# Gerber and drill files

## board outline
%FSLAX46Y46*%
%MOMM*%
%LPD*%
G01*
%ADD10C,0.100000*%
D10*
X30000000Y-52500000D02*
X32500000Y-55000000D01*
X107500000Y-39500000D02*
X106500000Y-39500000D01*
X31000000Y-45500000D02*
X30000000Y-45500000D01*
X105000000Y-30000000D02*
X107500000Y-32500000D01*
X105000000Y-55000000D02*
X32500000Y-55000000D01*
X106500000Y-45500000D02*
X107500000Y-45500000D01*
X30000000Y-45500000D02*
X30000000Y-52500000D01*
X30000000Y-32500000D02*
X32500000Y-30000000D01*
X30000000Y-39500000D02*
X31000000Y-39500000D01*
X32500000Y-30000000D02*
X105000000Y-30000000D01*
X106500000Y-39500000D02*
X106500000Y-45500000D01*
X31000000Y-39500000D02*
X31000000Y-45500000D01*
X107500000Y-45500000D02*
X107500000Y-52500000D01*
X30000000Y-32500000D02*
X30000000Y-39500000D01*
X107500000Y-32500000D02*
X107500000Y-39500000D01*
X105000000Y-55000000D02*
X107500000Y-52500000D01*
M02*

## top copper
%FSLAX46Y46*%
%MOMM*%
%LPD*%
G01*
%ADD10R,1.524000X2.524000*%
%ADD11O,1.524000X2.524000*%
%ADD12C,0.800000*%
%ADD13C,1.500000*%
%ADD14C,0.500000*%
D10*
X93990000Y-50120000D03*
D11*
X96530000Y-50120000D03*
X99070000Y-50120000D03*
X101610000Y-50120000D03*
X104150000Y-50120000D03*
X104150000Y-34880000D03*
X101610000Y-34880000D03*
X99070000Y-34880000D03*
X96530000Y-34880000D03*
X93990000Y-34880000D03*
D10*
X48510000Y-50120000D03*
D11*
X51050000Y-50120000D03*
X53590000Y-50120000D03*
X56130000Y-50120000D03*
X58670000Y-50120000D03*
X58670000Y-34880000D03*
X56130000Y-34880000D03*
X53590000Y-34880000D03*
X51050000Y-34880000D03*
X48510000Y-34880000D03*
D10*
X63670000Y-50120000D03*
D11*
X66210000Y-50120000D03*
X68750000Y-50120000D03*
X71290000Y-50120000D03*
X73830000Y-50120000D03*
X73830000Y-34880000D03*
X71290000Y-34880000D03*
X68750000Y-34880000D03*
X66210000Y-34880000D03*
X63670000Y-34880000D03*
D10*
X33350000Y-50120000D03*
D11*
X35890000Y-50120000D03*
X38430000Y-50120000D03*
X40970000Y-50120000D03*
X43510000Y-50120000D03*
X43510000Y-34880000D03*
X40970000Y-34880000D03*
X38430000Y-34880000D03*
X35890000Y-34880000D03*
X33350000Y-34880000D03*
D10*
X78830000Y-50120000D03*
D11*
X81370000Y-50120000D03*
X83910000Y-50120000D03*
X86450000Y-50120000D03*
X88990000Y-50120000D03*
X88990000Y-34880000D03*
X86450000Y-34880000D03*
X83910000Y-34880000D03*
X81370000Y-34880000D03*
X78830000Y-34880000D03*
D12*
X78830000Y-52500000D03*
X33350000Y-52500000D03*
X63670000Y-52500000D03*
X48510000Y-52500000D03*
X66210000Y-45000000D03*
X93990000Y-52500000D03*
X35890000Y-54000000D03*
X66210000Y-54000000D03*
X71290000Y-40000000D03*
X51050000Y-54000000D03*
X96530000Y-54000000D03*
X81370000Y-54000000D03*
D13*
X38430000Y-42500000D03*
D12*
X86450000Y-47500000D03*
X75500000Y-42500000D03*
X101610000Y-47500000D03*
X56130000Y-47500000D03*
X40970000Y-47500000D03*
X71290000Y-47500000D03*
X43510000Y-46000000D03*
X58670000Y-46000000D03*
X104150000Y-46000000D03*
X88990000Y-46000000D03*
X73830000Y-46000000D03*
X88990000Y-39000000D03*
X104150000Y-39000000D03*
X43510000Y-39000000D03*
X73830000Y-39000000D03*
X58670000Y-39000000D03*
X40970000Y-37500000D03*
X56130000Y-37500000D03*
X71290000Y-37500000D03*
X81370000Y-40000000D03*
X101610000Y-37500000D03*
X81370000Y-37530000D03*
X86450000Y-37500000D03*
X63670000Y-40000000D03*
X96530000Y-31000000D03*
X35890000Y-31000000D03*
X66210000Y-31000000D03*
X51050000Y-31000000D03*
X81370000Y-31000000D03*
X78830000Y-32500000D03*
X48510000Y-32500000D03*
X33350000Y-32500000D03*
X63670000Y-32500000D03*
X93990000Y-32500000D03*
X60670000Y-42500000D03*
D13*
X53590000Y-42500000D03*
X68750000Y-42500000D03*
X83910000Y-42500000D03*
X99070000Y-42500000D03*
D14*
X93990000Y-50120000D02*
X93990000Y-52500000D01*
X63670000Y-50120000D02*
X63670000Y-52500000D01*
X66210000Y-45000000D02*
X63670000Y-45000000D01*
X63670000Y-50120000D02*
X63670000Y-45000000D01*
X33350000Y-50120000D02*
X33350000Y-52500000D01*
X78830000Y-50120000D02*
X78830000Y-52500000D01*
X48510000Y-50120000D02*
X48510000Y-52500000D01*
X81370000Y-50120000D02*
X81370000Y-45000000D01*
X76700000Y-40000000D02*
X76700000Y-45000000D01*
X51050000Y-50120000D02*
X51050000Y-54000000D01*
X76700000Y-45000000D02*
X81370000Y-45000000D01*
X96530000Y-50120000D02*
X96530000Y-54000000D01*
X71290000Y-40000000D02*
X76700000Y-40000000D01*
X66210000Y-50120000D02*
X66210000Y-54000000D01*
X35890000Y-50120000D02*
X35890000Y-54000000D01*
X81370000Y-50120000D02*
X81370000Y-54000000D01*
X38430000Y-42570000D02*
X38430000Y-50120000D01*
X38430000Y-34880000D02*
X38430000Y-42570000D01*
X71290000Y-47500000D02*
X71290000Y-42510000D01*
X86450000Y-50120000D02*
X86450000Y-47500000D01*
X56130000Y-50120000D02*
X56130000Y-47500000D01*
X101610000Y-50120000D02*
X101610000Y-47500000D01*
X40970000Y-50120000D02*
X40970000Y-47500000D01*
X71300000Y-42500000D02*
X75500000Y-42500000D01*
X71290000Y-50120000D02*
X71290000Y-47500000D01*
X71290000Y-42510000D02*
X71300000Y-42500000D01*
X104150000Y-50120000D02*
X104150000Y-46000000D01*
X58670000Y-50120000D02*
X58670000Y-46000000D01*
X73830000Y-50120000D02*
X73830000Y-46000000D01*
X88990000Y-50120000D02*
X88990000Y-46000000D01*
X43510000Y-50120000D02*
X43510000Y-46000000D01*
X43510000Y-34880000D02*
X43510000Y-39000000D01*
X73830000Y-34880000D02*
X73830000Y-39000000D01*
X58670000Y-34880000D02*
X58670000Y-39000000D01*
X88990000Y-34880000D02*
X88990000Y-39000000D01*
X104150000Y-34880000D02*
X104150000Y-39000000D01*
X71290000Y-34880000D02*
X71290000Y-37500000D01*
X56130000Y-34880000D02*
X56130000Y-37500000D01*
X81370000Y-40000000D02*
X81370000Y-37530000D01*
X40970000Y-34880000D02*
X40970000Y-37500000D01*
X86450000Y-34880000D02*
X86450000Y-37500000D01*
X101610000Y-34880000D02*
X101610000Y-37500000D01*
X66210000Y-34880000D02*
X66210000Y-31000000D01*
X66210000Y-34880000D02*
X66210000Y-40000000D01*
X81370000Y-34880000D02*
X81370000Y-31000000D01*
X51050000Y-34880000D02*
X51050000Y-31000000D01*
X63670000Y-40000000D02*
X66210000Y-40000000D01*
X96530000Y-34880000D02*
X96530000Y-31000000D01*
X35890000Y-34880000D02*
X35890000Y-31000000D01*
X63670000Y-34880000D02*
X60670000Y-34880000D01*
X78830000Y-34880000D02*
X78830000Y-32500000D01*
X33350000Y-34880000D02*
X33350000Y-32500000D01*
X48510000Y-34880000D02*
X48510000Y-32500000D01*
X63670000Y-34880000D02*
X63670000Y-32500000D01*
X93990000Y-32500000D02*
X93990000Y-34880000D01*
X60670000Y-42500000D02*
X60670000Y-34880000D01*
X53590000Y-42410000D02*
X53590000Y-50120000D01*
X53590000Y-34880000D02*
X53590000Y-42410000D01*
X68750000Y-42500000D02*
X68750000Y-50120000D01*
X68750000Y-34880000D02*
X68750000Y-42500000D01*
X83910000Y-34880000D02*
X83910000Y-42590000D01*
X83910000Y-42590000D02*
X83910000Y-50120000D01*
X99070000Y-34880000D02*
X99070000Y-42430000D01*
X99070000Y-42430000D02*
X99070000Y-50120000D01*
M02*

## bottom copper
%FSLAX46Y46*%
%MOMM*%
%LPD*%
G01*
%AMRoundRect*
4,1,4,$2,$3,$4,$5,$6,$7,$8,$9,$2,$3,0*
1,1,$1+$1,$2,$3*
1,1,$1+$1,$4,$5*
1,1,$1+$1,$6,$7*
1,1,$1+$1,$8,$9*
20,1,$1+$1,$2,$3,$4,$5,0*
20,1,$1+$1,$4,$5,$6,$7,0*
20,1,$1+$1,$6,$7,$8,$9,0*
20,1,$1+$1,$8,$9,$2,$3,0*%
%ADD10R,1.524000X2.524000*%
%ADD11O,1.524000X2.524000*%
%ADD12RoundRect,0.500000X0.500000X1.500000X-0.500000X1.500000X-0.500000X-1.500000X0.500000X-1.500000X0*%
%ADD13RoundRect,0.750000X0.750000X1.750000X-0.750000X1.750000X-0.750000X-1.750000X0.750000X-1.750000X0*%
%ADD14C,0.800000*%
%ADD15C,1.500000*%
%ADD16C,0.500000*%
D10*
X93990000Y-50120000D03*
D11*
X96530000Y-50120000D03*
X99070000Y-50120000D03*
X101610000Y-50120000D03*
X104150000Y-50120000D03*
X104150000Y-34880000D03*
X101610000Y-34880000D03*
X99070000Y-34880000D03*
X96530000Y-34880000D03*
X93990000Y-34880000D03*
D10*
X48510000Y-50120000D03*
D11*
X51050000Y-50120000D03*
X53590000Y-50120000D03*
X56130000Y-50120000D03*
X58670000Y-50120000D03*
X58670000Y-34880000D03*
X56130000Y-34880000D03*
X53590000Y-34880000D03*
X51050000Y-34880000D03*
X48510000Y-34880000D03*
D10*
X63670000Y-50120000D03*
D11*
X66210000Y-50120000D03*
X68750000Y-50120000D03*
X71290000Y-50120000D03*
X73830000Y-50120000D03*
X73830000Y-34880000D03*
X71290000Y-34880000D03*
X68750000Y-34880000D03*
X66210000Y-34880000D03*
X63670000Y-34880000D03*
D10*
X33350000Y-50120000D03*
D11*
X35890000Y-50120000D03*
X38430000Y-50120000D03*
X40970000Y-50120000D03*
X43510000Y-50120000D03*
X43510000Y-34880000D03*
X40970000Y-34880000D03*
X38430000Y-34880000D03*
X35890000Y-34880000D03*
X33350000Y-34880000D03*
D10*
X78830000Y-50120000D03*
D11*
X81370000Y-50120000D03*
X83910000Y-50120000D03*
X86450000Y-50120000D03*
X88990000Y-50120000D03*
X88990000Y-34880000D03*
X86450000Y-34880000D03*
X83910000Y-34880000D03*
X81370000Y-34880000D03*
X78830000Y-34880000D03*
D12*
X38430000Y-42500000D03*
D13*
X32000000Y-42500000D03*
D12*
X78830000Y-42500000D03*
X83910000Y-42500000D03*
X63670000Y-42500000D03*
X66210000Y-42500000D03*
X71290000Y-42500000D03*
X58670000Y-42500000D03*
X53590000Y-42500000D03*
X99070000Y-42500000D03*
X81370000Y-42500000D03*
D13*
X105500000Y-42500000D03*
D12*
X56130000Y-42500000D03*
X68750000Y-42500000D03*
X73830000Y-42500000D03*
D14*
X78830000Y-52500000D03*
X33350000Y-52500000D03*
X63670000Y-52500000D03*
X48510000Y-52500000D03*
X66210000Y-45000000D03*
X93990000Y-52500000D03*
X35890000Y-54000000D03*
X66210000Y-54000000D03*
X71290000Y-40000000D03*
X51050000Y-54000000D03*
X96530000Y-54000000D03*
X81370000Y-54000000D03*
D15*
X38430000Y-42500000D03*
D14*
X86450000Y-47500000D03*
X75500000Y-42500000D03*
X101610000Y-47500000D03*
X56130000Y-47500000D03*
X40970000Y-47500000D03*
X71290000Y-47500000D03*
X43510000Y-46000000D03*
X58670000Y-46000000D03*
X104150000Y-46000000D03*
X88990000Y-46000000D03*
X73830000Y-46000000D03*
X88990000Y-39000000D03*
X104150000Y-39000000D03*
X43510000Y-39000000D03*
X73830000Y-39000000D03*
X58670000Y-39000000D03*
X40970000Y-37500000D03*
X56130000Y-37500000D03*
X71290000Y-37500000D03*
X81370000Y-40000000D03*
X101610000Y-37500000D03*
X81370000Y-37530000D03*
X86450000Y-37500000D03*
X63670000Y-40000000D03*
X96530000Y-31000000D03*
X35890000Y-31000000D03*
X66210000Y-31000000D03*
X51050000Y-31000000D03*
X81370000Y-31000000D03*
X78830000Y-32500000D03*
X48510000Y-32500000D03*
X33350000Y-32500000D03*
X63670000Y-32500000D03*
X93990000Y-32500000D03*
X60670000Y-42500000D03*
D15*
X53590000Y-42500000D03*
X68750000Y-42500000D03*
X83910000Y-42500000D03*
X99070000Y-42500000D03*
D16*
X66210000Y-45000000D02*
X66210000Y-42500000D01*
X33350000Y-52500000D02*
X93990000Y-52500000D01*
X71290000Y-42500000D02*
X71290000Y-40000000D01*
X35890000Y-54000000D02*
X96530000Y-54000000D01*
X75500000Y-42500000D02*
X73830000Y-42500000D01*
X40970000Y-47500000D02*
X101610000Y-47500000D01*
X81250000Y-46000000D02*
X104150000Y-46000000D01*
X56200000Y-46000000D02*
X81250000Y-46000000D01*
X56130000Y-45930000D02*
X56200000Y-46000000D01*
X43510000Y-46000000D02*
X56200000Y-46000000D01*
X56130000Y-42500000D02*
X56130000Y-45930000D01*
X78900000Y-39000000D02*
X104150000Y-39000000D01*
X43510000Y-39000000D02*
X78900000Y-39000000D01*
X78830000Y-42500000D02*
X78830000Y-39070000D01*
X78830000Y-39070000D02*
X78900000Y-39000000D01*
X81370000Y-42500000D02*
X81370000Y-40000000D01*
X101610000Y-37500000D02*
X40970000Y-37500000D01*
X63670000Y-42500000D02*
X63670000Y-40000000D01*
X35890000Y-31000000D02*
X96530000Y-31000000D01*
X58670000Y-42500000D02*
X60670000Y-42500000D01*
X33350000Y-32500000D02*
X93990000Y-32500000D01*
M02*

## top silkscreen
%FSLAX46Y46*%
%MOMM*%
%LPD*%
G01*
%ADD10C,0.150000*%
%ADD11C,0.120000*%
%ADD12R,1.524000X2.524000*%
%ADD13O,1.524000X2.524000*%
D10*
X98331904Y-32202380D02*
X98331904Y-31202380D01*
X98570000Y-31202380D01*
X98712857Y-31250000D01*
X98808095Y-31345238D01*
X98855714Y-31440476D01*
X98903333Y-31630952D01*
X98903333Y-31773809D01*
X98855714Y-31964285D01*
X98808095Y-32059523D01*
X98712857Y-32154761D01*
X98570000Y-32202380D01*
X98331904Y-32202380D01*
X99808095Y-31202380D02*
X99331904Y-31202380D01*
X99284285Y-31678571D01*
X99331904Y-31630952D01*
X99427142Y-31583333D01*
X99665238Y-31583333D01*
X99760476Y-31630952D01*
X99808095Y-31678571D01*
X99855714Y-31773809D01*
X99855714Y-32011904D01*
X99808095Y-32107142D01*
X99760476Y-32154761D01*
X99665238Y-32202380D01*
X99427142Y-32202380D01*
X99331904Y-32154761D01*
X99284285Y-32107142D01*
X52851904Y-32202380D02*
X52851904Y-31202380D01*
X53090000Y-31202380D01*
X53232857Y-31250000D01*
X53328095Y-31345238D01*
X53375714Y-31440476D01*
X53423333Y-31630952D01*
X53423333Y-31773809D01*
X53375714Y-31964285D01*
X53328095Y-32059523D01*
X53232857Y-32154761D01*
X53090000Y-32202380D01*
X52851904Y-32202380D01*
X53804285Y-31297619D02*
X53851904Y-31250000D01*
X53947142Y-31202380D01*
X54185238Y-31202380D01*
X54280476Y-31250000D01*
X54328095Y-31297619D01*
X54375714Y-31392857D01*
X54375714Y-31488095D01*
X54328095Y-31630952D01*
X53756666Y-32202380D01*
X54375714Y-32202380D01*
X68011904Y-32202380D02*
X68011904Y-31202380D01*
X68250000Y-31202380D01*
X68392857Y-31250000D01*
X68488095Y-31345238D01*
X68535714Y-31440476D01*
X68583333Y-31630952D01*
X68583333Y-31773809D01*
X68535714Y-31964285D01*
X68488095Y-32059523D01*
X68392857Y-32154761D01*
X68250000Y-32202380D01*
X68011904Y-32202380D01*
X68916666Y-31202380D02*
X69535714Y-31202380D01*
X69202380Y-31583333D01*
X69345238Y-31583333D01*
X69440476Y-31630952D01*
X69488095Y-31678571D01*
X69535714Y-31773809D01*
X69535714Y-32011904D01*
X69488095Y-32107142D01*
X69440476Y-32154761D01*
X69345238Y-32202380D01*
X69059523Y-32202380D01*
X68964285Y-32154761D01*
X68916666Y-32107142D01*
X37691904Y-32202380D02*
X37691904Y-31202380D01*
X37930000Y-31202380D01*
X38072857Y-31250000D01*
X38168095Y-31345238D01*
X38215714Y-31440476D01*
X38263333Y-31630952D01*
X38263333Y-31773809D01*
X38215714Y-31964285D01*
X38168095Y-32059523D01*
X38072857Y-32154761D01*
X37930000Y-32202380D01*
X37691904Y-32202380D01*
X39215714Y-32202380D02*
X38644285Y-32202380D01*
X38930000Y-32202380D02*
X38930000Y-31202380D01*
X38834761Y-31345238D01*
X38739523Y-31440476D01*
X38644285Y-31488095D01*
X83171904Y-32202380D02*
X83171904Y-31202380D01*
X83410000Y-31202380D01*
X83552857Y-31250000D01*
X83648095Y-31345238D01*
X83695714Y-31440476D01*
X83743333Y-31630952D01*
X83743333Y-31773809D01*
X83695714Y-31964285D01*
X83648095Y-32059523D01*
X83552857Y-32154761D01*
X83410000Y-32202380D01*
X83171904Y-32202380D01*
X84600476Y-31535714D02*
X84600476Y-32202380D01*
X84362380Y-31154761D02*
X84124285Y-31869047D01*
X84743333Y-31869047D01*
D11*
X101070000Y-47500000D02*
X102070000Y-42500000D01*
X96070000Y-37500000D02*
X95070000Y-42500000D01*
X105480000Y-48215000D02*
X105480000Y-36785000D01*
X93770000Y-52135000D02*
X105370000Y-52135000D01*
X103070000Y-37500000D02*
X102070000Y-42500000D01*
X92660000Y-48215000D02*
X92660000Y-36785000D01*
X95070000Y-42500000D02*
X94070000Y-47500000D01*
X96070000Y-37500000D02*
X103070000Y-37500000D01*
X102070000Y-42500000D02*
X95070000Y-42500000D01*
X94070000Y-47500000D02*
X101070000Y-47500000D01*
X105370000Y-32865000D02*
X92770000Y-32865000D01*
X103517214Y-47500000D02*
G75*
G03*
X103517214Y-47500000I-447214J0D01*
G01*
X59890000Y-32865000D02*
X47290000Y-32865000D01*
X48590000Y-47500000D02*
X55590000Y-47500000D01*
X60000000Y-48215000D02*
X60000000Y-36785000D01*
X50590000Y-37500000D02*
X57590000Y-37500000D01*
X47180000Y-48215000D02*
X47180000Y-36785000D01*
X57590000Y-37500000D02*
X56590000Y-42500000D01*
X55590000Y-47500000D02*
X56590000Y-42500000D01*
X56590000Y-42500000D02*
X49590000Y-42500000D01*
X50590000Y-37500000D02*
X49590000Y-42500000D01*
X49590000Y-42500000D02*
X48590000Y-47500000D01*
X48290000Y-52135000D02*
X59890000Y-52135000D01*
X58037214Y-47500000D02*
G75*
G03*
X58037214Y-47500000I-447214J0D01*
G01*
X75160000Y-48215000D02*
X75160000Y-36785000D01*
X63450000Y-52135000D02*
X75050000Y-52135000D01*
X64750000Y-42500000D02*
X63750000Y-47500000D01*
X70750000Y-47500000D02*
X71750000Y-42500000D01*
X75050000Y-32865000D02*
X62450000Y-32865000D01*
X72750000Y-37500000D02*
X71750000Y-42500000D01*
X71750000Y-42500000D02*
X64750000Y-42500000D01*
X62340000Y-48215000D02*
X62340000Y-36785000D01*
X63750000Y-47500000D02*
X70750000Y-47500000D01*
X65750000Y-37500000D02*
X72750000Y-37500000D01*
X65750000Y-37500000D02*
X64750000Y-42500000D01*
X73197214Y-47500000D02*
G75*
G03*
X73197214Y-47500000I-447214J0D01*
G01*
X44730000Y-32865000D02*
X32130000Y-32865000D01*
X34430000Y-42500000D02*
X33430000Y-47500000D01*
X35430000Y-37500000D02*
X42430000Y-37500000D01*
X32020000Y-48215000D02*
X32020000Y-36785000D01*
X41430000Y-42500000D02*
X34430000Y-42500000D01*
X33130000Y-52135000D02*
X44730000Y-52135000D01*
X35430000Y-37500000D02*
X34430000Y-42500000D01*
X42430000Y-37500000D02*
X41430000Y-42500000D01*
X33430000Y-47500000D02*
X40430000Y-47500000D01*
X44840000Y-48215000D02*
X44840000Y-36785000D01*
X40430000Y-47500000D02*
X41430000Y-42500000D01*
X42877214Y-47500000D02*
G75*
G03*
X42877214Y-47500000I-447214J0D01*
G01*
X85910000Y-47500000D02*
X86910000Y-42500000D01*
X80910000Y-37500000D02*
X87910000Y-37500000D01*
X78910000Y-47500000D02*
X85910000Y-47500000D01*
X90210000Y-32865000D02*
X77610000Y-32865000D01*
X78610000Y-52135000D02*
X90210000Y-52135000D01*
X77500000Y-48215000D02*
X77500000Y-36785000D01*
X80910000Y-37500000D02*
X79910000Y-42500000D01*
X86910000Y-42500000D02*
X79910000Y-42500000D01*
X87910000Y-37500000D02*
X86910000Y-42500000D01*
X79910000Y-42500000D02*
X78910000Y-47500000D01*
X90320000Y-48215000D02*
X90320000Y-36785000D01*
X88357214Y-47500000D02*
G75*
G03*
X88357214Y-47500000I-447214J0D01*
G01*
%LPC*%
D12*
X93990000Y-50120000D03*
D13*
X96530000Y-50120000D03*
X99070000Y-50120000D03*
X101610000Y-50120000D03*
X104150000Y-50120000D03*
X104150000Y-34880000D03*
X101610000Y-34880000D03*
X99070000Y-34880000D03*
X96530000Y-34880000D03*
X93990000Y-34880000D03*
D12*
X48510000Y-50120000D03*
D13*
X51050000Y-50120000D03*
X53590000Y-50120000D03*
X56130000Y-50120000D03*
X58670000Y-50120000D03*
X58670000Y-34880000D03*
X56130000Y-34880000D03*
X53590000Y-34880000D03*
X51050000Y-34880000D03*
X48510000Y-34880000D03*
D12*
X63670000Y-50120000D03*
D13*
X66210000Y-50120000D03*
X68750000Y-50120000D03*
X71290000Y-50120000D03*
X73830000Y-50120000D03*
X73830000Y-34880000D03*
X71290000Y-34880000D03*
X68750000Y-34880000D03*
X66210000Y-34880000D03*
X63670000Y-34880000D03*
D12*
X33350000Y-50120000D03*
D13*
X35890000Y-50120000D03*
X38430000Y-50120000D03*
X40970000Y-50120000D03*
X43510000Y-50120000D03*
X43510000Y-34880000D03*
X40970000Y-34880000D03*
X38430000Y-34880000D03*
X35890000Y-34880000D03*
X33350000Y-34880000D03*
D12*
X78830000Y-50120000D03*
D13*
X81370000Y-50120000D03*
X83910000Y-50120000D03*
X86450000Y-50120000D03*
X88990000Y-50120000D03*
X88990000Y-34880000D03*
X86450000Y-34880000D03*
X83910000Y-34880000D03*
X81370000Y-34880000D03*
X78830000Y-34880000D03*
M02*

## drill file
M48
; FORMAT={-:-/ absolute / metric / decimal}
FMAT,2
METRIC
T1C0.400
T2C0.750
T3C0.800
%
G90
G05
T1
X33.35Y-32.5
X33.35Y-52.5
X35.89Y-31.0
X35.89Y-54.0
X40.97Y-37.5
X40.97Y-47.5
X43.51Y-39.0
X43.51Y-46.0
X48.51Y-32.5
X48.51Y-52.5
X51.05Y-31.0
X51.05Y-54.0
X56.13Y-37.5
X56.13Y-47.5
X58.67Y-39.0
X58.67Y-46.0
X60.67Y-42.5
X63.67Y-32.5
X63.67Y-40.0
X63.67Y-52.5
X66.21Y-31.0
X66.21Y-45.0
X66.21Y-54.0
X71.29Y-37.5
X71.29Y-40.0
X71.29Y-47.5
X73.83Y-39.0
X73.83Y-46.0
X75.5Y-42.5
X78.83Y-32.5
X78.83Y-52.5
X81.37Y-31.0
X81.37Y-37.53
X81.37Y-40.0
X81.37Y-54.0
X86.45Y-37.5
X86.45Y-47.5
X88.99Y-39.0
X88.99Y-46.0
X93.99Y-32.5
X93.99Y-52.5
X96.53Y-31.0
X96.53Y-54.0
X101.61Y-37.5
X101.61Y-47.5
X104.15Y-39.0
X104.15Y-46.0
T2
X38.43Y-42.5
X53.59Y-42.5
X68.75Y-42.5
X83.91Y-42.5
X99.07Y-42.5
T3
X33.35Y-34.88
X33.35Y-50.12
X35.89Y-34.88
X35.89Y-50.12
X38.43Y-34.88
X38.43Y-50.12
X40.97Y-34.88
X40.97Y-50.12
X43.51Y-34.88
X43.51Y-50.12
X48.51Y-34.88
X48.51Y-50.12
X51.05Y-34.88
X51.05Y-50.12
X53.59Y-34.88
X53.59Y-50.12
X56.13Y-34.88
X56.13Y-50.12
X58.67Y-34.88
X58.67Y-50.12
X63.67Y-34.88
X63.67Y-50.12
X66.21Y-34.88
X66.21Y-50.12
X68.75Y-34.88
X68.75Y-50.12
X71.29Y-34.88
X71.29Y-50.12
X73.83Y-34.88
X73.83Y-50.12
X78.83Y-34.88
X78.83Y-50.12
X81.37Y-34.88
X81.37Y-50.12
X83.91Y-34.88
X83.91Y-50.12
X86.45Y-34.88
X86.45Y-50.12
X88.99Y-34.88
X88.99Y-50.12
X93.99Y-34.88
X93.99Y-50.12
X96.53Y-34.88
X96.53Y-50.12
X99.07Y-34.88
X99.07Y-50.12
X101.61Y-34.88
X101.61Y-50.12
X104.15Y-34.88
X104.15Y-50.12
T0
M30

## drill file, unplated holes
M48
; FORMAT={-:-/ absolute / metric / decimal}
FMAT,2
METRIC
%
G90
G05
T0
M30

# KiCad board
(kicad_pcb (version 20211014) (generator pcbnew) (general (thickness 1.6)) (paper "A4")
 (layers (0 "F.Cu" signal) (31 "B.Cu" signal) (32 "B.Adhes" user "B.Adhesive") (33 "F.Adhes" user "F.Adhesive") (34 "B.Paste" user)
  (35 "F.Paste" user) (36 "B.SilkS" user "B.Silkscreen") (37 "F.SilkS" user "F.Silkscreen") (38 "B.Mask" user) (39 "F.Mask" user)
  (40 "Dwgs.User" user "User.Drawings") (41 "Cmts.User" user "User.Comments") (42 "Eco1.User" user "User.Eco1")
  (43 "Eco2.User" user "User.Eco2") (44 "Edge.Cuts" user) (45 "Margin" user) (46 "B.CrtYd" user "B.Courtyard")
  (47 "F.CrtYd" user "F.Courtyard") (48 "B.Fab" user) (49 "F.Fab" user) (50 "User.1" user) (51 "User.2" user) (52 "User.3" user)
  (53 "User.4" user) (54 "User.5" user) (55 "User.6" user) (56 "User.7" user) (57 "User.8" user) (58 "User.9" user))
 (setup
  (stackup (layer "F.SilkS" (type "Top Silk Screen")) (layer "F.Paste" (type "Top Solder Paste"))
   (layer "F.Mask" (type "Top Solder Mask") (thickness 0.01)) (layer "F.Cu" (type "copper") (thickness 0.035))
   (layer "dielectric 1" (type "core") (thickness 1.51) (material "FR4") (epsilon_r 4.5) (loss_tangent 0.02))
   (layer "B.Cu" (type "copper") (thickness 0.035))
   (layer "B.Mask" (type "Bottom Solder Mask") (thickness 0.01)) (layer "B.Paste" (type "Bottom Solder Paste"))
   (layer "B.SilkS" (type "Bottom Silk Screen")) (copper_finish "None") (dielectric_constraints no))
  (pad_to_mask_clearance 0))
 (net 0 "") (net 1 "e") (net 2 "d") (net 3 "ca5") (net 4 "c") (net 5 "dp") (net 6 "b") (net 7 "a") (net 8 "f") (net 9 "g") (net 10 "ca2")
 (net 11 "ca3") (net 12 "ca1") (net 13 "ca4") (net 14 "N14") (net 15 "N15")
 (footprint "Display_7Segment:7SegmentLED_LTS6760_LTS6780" (layer "F.Cu") (at 93.99 50.12 90)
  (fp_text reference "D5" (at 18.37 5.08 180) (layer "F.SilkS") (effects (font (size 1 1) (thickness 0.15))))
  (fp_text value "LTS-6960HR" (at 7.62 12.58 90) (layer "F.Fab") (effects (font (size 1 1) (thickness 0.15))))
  (fp_line (start 2.62 7.08) (end 7.62 8.08) (layer "F.SilkS") (width 0.12))
  (fp_line (start 12.62 2.08) (end 7.62 1.08) (layer "F.SilkS") (width 0.12))
  (fp_line (start 1.905 11.49) (end 13.335 11.49) (layer "F.SilkS") (width 0.12))
  (fp_line (start -2.015 -0.22) (end -2.015 11.38) (layer "F.SilkS") (width 0.12))
  (fp_line (start 12.62 9.08) (end 7.62 8.08) (layer "F.SilkS") (width 0.12))
  (fp_line (start 1.905 -1.33) (end 13.335 -1.33) (layer "F.SilkS") (width 0.12))
  (fp_line (start 7.62 1.08) (end 2.62 0.08) (layer "F.SilkS") (width 0.12))
  (fp_line (start 12.62 2.08) (end 12.62 9.08) (layer "F.SilkS") (width 0.12))
  (fp_line (start 7.62 8.08) (end 7.62 1.08) (layer "F.SilkS") (width 0.12))
  (fp_line (start 2.62 0.08) (end 2.62 7.08) (layer "F.SilkS") (width 0.12))
  (fp_line (start 17.255 11.38) (end 17.255 -1.22) (layer "F.SilkS") (width 0.12))
  (fp_circle (center 2.62 9.08) (end 3.067214 9.08) (layer "F.SilkS") (width 0.12) (fill none))
  (pad "1" thru_hole rect (at 0 0) (size 1.524 2.524) (drill 0.8) (layers *.Cu *.Mask) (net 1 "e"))
  (pad "2" thru_hole oval (at 0 2.54) (size 1.524 2.524) (drill 0.8) (layers *.Cu *.Mask) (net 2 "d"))
  (pad "3" thru_hole oval (at 0 5.08) (size 1.524 2.524) (drill 0.8) (layers *.Cu *.Mask) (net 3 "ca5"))
  (pad "4" thru_hole oval (at 0 7.62) (size 1.524 2.524) (drill 0.8) (layers *.Cu *.Mask) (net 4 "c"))
  (pad "5" thru_hole oval (at 0 10.16) (size 1.524 2.524) (drill 0.8) (layers *.Cu *.Mask) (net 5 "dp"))
  (pad "6" thru_hole oval (at 15.24 10.16) (size 1.524 2.524) (drill 0.8) (layers *.Cu *.Mask) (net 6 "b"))
  (pad "7" thru_hole oval (at 15.24 7.62) (size 1.524 2.524) (drill 0.8) (layers *.Cu *.Mask) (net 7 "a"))
  (pad "8" thru_hole oval (at 15.24 5.08) (size 1.524 2.524) (drill 0.8) (layers *.Cu *.Mask) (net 3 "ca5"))
  (pad "9" thru_hole oval (at 15.24 2.54) (size 1.524 2.524) (drill 0.8) (layers *.Cu *.Mask) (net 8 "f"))
  (pad "10" thru_hole oval (at 15.24 0) (size 1.524 2.524) (drill 0.8) (layers *.Cu *.Mask) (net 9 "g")))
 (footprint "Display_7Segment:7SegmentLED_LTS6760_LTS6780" (layer "F.Cu") (at 48.51 50.12 90)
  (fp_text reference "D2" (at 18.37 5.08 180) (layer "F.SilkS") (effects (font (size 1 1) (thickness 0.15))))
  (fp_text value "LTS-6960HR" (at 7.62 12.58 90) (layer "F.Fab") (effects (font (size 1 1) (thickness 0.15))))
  (fp_line (start 17.255 11.38) (end 17.255 -1.22) (layer "F.SilkS") (width 0.12))
  (fp_line (start 2.62 0.08) (end 2.62 7.08) (layer "F.SilkS") (width 0.12))
  (fp_line (start 1.905 11.49) (end 13.335 11.49) (layer "F.SilkS") (width 0.12))
  (fp_line (start 12.62 2.08) (end 12.62 9.08) (layer "F.SilkS") (width 0.12))
  (fp_line (start 1.905 -1.33) (end 13.335 -1.33) (layer "F.SilkS") (width 0.12))
  (fp_line (start 12.62 9.08) (end 7.62 8.08) (layer "F.SilkS") (width 0.12))
  (fp_line (start 2.62 7.08) (end 7.62 8.08) (layer "F.SilkS") (width 0.12))
  (fp_line (start 7.62 8.08) (end 7.62 1.08) (layer "F.SilkS") (width 0.12))
  (fp_line (start 12.62 2.08) (end 7.62 1.08) (layer "F.SilkS") (width 0.12))
  (fp_line (start 7.62 1.08) (end 2.62 0.08) (layer "F.SilkS") (width 0.12))
  (fp_line (start -2.015 -0.22) (end -2.015 11.38) (layer "F.SilkS") (width 0.12))
  (fp_circle (center 2.62 9.08) (end 3.067214 9.08) (layer "F.SilkS") (width 0.12) (fill none))
  (pad "1" thru_hole rect (at 0 0) (size 1.524 2.524) (drill 0.8) (layers *.Cu *.Mask) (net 1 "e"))
  (pad "2" thru_hole oval (at 0 2.54) (size 1.524 2.524) (drill 0.8) (layers *.Cu *.Mask) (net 2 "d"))
  (pad "3" thru_hole oval (at 0 5.08) (size 1.524 2.524) (drill 0.8) (layers *.Cu *.Mask) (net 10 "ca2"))
  (pad "4" thru_hole oval (at 0 7.62) (size 1.524 2.524) (drill 0.8) (layers *.Cu *.Mask) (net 4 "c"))
  (pad "5" thru_hole oval (at 0 10.16) (size 1.524 2.524) (drill 0.8) (layers *.Cu *.Mask) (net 5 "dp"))
  (pad "6" thru_hole oval (at 15.24 10.16) (size 1.524 2.524) (drill 0.8) (layers *.Cu *.Mask) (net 6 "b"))
  (pad "7" thru_hole oval (at 15.24 7.62) (size 1.524 2.524) (drill 0.8) (layers *.Cu *.Mask) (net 7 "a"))
  (pad "8" thru_hole oval (at 15.24 5.08) (size 1.524 2.524) (drill 0.8) (layers *.Cu *.Mask) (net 10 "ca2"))
  (pad "9" thru_hole oval (at 15.24 2.54) (size 1.524 2.524) (drill 0.8) (layers *.Cu *.Mask) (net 8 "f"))
  (pad "10" thru_hole oval (at 15.24 0) (size 1.524 2.524) (drill 0.8) (layers *.Cu *.Mask) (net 9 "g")))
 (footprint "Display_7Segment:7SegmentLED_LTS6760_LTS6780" (layer "F.Cu") (at 63.67 50.12 90)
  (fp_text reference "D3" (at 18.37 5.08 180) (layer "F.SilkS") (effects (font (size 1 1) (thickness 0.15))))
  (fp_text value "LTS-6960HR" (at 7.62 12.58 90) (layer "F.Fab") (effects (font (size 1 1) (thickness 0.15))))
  (fp_line (start 1.905 11.49) (end 13.335 11.49) (layer "F.SilkS") (width 0.12))
  (fp_line (start -2.015 -0.22) (end -2.015 11.38) (layer "F.SilkS") (width 0.12))
  (fp_line (start 7.62 1.08) (end 2.62 0.08) (layer "F.SilkS") (width 0.12))
  (fp_line (start 2.62 7.08) (end 7.62 8.08) (layer "F.SilkS") (width 0.12))
  (fp_line (start 17.255 11.38) (end 17.255 -1.22) (layer "F.SilkS") (width 0.12))
  (fp_line (start 12.62 9.08) (end 7.62 8.08) (layer "F.SilkS") (width 0.12))
  (fp_line (start 7.62 8.08) (end 7.62 1.08) (layer "F.SilkS") (width 0.12))
  (fp_line (start 1.905 -1.33) (end 13.335 -1.33) (layer "F.SilkS") (width 0.12))
  (fp_line (start 2.62 0.08) (end 2.62 7.08) (layer "F.SilkS") (width 0.12))
  (fp_line (start 12.62 2.08) (end 12.62 9.08) (layer "F.SilkS") (width 0.12))
  (fp_line (start 12.62 2.08) (end 7.62 1.08) (layer "F.SilkS") (width 0.12))
  (fp_circle (center 2.62 9.08) (end 3.067214 9.08) (layer "F.SilkS") (width 0.12) (fill none))
  (pad "1" thru_hole rect (at 0 0) (size 1.524 2.524) (drill 0.8) (layers *.Cu *.Mask) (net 1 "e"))
  (pad "2" thru_hole oval (at 0 2.54) (size 1.524 2.524) (drill 0.8) (layers *.Cu *.Mask) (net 2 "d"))
  (pad "3" thru_hole oval (at 0 5.08) (size 1.524 2.524) (drill 0.8) (layers *.Cu *.Mask) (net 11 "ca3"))
  (pad "4" thru_hole oval (at 0 7.62) (size 1.524 2.524) (drill 0.8) (layers *.Cu *.Mask) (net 4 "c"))
  (pad "5" thru_hole oval (at 0 10.16) (size 1.524 2.524) (drill 0.8) (layers *.Cu *.Mask) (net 5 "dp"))
  (pad "6" thru_hole oval (at 15.24 10.16) (size 1.524 2.524) (drill 0.8) (layers *.Cu *.Mask) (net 6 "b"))
  (pad "7" thru_hole oval (at 15.24 7.62) (size 1.524 2.524) (drill 0.8) (layers *.Cu *.Mask) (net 7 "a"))
  (pad "8" thru_hole oval (at 15.24 5.08) (size 1.524 2.524) (drill 0.8) (layers *.Cu *.Mask) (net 11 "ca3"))
  (pad "9" thru_hole oval (at 15.24 2.54) (size 1.524 2.524) (drill 0.8) (layers *.Cu *.Mask) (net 8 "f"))
  (pad "10" thru_hole oval (at 15.24 0) (size 1.524 2.524) (drill 0.8) (layers *.Cu *.Mask) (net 9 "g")))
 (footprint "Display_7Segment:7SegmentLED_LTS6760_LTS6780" (layer "F.Cu") (at 33.35 50.12 90)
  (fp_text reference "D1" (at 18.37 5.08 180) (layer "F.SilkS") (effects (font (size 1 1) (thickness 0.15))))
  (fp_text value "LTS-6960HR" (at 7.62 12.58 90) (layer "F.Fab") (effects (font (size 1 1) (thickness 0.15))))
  (fp_line (start 17.255 11.38) (end 17.255 -1.22) (layer "F.SilkS") (width 0.12))
  (fp_line (start 7.62 1.08) (end 2.62 0.08) (layer "F.SilkS") (width 0.12))
  (fp_line (start 12.62 2.08) (end 12.62 9.08) (layer "F.SilkS") (width 0.12))
  (fp_line (start 1.905 -1.33) (end 13.335 -1.33) (layer "F.SilkS") (width 0.12))
  (fp_line (start 7.62 8.08) (end 7.62 1.08) (layer "F.SilkS") (width 0.12))
  (fp_line (start -2.015 -0.22) (end -2.015 11.38) (layer "F.SilkS") (width 0.12))
  (fp_line (start 12.62 2.08) (end 7.62 1.08) (layer "F.SilkS") (width 0.12))
  (fp_line (start 12.62 9.08) (end 7.62 8.08) (layer "F.SilkS") (width 0.12))
  (fp_line (start 2.62 0.08) (end 2.62 7.08) (layer "F.SilkS") (width 0.12))
  (fp_line (start 1.905 11.49) (end 13.335 11.49) (layer "F.SilkS") (width 0.12))
  (fp_line (start 2.62 7.08) (end 7.62 8.08) (layer "F.SilkS") (width 0.12))
  (fp_circle (center 2.62 9.08) (end 3.067214 9.08) (layer "F.SilkS") (width 0.12) (fill none))
  (pad "1" thru_hole rect (at 0 0) (size 1.524 2.524) (drill 0.8) (layers *.Cu *.Mask) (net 1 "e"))
  (pad "2" thru_hole oval (at 0 2.54) (size 1.524 2.524) (drill 0.8) (layers *.Cu *.Mask) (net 2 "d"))
  (pad "3" thru_hole oval (at 0 5.08) (size 1.524 2.524) (drill 0.8) (layers *.Cu *.Mask) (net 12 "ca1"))
  (pad "4" thru_hole oval (at 0 7.62) (size 1.524 2.524) (drill 0.8) (layers *.Cu *.Mask) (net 4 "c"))
  (pad "5" thru_hole oval (at 0 10.16) (size 1.524 2.524) (drill 0.8) (layers *.Cu *.Mask) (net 5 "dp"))
  (pad "6" thru_hole oval (at 15.24 10.16) (size 1.524 2.524) (drill 0.8) (layers *.Cu *.Mask) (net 6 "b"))
  (pad "7" thru_hole oval (at 15.24 7.62) (size 1.524 2.524) (drill 0.8) (layers *.Cu *.Mask) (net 7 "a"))
  (pad "8" thru_hole oval (at 15.24 5.08) (size 1.524 2.524) (drill 0.8) (layers *.Cu *.Mask) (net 12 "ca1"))
  (pad "9" thru_hole oval (at 15.24 2.54) (size 1.524 2.524) (drill 0.8) (layers *.Cu *.Mask) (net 8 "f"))
  (pad "10" thru_hole oval (at 15.24 0) (size 1.524 2.524) (drill 0.8) (layers *.Cu *.Mask) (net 9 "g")))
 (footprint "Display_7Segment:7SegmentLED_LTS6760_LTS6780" (layer "F.Cu") (at 78.83 50.12 90)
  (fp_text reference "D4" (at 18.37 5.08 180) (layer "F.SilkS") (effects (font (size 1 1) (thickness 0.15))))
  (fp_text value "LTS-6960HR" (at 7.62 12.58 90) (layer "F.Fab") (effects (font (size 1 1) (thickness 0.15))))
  (fp_line (start 2.62 7.08) (end 7.62 8.08) (layer "F.SilkS") (width 0.12))
  (fp_line (start 12.62 2.08) (end 12.62 9.08) (layer "F.SilkS") (width 0.12))
  (fp_line (start 2.62 0.08) (end 2.62 7.08) (layer "F.SilkS") (width 0.12))
  (fp_line (start 17.255 11.38) (end 17.255 -1.22) (layer "F.SilkS") (width 0.12))
  (fp_line (start -2.015 -0.22) (end -2.015 11.38) (layer "F.SilkS") (width 0.12))
  (fp_line (start 1.905 -1.33) (end 13.335 -1.33) (layer "F.SilkS") (width 0.12))
  (fp_line (start 12.62 2.08) (end 7.62 1.08) (layer "F.SilkS") (width 0.12))
  (fp_line (start 7.62 8.08) (end 7.62 1.08) (layer "F.SilkS") (width 0.12))
  (fp_line (start 12.62 9.08) (end 7.62 8.08) (layer "F.SilkS") (width 0.12))
  (fp_line (start 7.62 1.08) (end 2.62 0.08) (layer "F.SilkS") (width 0.12))
  (fp_line (start 1.905 11.49) (end 13.335 11.49) (layer "F.SilkS") (width 0.12))
  (fp_circle (center 2.62 9.08) (end 3.067214 9.08) (layer "F.SilkS") (width 0.12) (fill none))
  (pad "1" thru_hole rect (at 0 0) (size 1.524 2.524) (drill 0.8) (layers *.Cu *.Mask) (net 1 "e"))
  (pad "2" thru_hole oval (at 0 2.54) (size 1.524 2.524) (drill 0.8) (layers *.Cu *.Mask) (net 2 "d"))
  (pad "3" thru_hole oval (at 0 5.08) (size 1.524 2.524) (drill 0.8) (layers *.Cu *.Mask) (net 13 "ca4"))
  (pad "4" thru_hole oval (at 0 7.62) (size 1.524 2.524) (drill 0.8) (layers *.Cu *.Mask) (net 4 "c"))
  (pad "5" thru_hole oval (at 0 10.16) (size 1.524 2.524) (drill 0.8) (layers *.Cu *.Mask) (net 5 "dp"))
  (pad "6" thru_hole oval (at 15.24 10.16) (size 1.524 2.524) (drill 0.8) (layers *.Cu *.Mask) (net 6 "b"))
  (pad "7" thru_hole oval (at 15.24 7.62) (size 1.524 2.524) (drill 0.8) (layers *.Cu *.Mask) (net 7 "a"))
  (pad "8" thru_hole oval (at 15.24 5.08) (size 1.524 2.524) (drill 0.8) (layers *.Cu *.Mask) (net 13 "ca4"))
  (pad "9" thru_hole oval (at 15.24 2.54) (size 1.524 2.524) (drill 0.8) (layers *.Cu *.Mask) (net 8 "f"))
  (pad "10" thru_hole oval (at 15.24 0) (size 1.524 2.524) (drill 0.8) (layers *.Cu *.Mask) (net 9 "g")))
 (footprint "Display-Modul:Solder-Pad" (layer "B.Cu") (at 38.43 42.5 180)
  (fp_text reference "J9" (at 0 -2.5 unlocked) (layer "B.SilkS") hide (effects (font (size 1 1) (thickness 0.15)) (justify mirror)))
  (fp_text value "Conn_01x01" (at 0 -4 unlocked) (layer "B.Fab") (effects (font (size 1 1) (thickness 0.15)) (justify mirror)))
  (pad "1" smd roundrect (at 0 0 180) (size 2 4) (layers "B.Cu" "B.Paste" "B.Mask") (roundrect_rratio 0.25) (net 12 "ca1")))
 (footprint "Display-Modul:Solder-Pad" (layer "B.Cu") (at 32 42.5 180)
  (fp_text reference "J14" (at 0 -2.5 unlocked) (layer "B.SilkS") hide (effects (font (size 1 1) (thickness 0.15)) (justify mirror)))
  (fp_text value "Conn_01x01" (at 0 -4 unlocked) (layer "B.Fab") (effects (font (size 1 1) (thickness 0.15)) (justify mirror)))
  (pad "1" smd roundrect (at 0 0 180) (size 3 5) (layers "B.Cu" "B.Paste" "B.Mask") (roundrect_rratio 0.25) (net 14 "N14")))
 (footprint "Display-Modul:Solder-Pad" (layer "B.Cu") (at 78.83 42.5 180)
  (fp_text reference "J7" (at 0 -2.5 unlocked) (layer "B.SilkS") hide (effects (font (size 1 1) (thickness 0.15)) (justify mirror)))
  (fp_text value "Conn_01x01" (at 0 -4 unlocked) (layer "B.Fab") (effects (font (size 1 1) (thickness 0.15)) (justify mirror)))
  (pad "1" smd roundrect (at 0 0 180) (size 2 4) (layers "B.Cu" "B.Paste" "B.Mask") (roundrect_rratio 0.25) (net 6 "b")))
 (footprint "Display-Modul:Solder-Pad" (layer "B.Cu") (at 83.91 42.5 180)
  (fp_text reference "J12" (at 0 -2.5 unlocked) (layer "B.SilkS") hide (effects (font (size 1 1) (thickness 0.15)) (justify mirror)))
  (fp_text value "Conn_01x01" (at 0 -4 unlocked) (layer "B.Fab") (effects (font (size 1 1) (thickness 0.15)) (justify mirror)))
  (pad "1" smd roundrect (at 0 0 180) (size 2 4) (layers "B.Cu" "B.Paste" "B.Mask") (roundrect_rratio 0.25) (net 13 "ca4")))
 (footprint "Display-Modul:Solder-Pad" (layer "B.Cu") (at 63.67 42.5 180)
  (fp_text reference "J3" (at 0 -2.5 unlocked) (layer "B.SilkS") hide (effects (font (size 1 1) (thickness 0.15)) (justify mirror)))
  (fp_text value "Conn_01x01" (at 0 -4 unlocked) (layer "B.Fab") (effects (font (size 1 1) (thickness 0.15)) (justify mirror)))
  (pad "1" smd roundrect (at 0 0 180) (size 2 4) (layers "B.Cu" "B.Paste" "B.Mask") (roundrect_rratio 0.25) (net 8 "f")))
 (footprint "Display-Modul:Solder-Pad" (layer "B.Cu") (at 66.21 42.5 180)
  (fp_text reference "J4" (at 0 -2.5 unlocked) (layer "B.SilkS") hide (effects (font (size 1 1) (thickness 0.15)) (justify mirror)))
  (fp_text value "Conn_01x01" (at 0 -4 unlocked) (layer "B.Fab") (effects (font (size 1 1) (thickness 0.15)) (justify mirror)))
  (pad "1" smd roundrect (at 0 0 180) (size 2 4) (layers "B.Cu" "B.Paste" "B.Mask") (roundrect_rratio 0.25) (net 1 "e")))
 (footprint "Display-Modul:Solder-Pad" (layer "B.Cu") (at 71.29 42.5 180)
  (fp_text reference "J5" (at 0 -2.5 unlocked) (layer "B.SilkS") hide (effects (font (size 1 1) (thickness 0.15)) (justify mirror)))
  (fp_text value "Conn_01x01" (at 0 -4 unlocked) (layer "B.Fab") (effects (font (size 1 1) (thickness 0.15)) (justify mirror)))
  (pad "1" smd roundrect (at 0 0 180) (size 2 4) (layers "B.Cu" "B.Paste" "B.Mask") (roundrect_rratio 0.25) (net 2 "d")))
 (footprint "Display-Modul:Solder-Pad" (layer "B.Cu") (at 58.67 42.5 180)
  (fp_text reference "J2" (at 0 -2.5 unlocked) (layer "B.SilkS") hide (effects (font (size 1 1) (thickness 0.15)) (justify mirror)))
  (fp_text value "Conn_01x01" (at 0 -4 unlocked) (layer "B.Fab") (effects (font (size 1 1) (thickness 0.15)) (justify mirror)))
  (pad "1" smd roundrect (at 0 0 180) (size 2 4) (layers "B.Cu" "B.Paste" "B.Mask") (roundrect_rratio 0.25) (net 9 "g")))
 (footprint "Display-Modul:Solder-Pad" (layer "B.Cu") (at 53.59 42.5 180)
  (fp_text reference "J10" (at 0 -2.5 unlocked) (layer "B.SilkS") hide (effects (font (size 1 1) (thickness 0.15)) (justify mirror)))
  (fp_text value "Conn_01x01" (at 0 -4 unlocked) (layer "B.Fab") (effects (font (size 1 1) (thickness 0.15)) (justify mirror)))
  (pad "1" smd roundrect (at 0 0 180) (size 2 4) (layers "B.Cu" "B.Paste" "B.Mask") (roundrect_rratio 0.25) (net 10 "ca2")))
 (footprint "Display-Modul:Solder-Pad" (layer "B.Cu") (at 99.07 42.5 180)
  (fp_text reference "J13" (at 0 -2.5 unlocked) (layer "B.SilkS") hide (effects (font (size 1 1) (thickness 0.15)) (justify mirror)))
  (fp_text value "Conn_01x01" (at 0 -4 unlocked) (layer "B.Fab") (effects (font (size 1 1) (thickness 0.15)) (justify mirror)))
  (pad "1" smd roundrect (at 0 0 180) (size 2 4) (layers "B.Cu" "B.Paste" "B.Mask") (roundrect_rratio 0.25) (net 3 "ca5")))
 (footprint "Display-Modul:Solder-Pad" (layer "B.Cu") (at 81.37 42.5 180)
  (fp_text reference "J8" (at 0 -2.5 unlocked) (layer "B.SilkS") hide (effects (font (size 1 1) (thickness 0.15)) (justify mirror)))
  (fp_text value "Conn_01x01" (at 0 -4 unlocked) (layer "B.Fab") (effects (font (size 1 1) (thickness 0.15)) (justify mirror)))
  (pad "1" smd roundrect (at 0 0 180) (size 2 4) (layers "B.Cu" "B.Paste" "B.Mask") (roundrect_rratio 0.25) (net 7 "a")))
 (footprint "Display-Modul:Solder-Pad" (layer "B.Cu") (at 105.5 42.5 180)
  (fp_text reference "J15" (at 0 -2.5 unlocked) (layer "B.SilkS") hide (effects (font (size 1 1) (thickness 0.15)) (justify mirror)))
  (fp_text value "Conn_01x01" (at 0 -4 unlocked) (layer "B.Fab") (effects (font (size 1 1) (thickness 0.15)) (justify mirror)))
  (pad "1" smd roundrect (at 0 0 180) (size 3 5) (layers "B.Cu" "B.Paste" "B.Mask") (roundrect_rratio 0.25) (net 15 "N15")))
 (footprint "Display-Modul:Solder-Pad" (layer "B.Cu") (at 56.13 42.5 180)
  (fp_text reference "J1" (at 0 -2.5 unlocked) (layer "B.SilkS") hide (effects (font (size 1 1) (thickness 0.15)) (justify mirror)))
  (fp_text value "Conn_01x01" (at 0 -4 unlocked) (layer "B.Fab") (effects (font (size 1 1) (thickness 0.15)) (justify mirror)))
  (pad "1" smd roundrect (at 0 0 180) (size 2 4) (layers "B.Cu" "B.Paste" "B.Mask") (roundrect_rratio 0.25) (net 5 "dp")))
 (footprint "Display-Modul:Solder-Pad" (layer "B.Cu") (at 68.75 42.5 180)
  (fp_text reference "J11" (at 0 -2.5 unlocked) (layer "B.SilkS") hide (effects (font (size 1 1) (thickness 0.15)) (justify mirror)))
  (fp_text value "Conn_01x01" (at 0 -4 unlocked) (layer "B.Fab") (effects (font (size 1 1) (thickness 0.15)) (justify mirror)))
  (pad "1" smd roundrect (at 0 0 180) (size 2 4) (layers "B.Cu" "B.Paste" "B.Mask") (roundrect_rratio 0.25) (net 11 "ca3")))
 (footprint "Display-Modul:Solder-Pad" (layer "B.Cu") (at 73.83 42.5 180)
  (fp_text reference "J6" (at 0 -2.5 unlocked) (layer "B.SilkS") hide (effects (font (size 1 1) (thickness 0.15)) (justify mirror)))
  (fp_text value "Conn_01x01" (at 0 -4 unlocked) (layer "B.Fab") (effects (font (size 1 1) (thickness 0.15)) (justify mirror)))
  (pad "1" smd roundrect (at 0 0 180) (size 2 4) (layers "B.Cu" "B.Paste" "B.Mask") (roundrect_rratio 0.25) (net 4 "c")))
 (gr_line (start 30 52.5) (end 32.5 55) (layer "Edge.Cuts") (width 0.1))
 (gr_line (start 107.5 39.5) (end 106.5 39.5) (layer "Edge.Cuts") (width 0.1))
 (gr_line (start 31 45.5) (end 30 45.5) (layer "Edge.Cuts") (width 0.1))
 (gr_line (start 105 30) (end 107.5 32.5) (layer "Edge.Cuts") (width 0.1))
 (gr_line (start 105 55) (end 32.5 55) (layer "Edge.Cuts") (width 0.1))
 (gr_line (start 106.5 45.5) (end 107.5 45.5) (layer "Edge.Cuts") (width 0.1))
 (gr_line (start 30 45.5) (end 30 52.5) (layer "Edge.Cuts") (width 0.1))
 (gr_line (start 30 32.5) (end 32.5 30) (layer "Edge.Cuts") (width 0.1))
 (gr_line (start 30 39.5) (end 31 39.5) (layer "Edge.Cuts") (width 0.1))
 (gr_line (start 32.5 30) (end 105 30) (layer "Edge.Cuts") (width 0.1))
 (gr_line (start 106.5 39.5) (end 106.5 45.5) (layer "Edge.Cuts") (width 0.1))
 (gr_line (start 31 39.5) (end 31 45.5) (layer "Edge.Cuts") (width 0.1))
 (gr_line (start 107.5 45.5) (end 107.5 52.5) (layer "Edge.Cuts") (width 0.1))
 (gr_line (start 30 32.5) (end 30 39.5) (layer "Edge.Cuts") (width 0.1))
 (gr_line (start 107.5 32.5) (end 107.5 39.5) (layer "Edge.Cuts") (width 0.1))
 (gr_line (start 105 55) (end 107.5 52.5) (layer "Edge.Cuts") (width 0.1))
 (segment (start 93.99 50.12) (end 93.99 52.5) (width 0.5) (layer "F.Cu") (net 1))
 (segment (start 63.67 50.12) (end 63.67 52.5) (width 0.5) (layer "F.Cu") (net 1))
 (segment (start 66.21 45) (end 63.67 45) (width 0.5) (layer "F.Cu") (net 1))
 (segment (start 63.67 50.12) (end 63.67 45) (width 0.5) (layer "F.Cu") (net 1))
 (segment (start 33.35 50.12) (end 33.35 52.5) (width 0.5) (layer "F.Cu") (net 1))
 (segment (start 78.83 50.12) (end 78.83 52.5) (width 0.5) (layer "F.Cu") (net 1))
 (segment (start 48.51 50.12) (end 48.51 52.5) (width 0.5) (layer "F.Cu") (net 1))
 (via (at 78.83 52.5) (size 0.8) (drill 0.4) (layers "F.Cu" "B.Cu") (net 1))
 (via (at 33.35 52.5) (size 0.8) (drill 0.4) (layers "F.Cu" "B.Cu") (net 1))
 (via (at 63.67 52.5) (size 0.8) (drill 0.4) (layers "F.Cu" "B.Cu") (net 1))
 (via (at 48.51 52.5) (size 0.8) (drill 0.4) (layers "F.Cu" "B.Cu") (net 1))
 (via (at 66.21 45) (size 0.8) (drill 0.4) (layers "F.Cu" "B.Cu") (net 1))
 (via (at 93.99 52.5) (size 0.8) (drill 0.4) (layers "F.Cu" "B.Cu") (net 1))
 (segment (start 66.21 45) (end 66.21 42.5) (width 0.5) (layer "B.Cu") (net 1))
 (segment (start 33.35 52.5) (end 93.99 52.5) (width 0.5) (layer "B.Cu") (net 1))
 (segment (start 81.37 50.12) (end 81.37 45) (width 0.5) (layer "F.Cu") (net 2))
 (segment (start 76.7 40) (end 76.7 45) (width 0.5) (layer "F.Cu") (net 2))
 (segment (start 51.05 50.12) (end 51.05 54) (width 0.5) (layer "F.Cu") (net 2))
 (segment (start 76.7 45) (end 81.37 45) (width 0.5) (layer "F.Cu") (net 2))
 (segment (start 96.53 50.12) (end 96.53 54) (width 0.5) (layer "F.Cu") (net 2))
 (segment (start 71.29 40) (end 76.7 40) (width 0.5) (layer "F.Cu") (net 2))
 (segment (start 66.21 50.12) (end 66.21 54) (width 0.5) (layer "F.Cu") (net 2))
 (segment (start 35.89 50.12) (end 35.89 54) (width 0.5) (layer "F.Cu") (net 2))
 (segment (start 81.37 50.12) (end 81.37 54) (width 0.5) (layer "F.Cu") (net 2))
 (via (at 35.89 54) (size 0.8) (drill 0.4) (layers "F.Cu" "B.Cu") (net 2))
 (via (at 66.21 54) (size 0.8) (drill 0.4) (layers "F.Cu" "B.Cu") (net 2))
 (via (at 71.29 40) (size 0.8) (drill 0.4) (layers "F.Cu" "B.Cu") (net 2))
 (via (at 51.05 54) (size 0.8) (drill 0.4) (layers "F.Cu" "B.Cu") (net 2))
 (via (at 96.53 54) (size 0.8) (drill 0.4) (layers "F.Cu" "B.Cu") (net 2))
 (via (at 81.37 54) (size 0.8) (drill 0.4) (layers "F.Cu" "B.Cu") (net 2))
 (segment (start 71.29 42.5) (end 71.29 40) (width 0.5) (layer "B.Cu") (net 2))
 (segment (start 35.89 54) (end 96.53 54) (width 0.5) (layer "B.Cu") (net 2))
 (segment (start 38.43 42.57) (end 38.43 50.12) (width 0.5) (layer "F.Cu") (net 12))
 (segment (start 38.43 34.88) (end 38.43 42.57) (width 0.5) (layer "F.Cu") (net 12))
 (via (at 38.43 42.5) (size 1.5) (drill 0.75) (layers "F.Cu" "B.Cu") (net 12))
 (segment (start 71.29 47.5) (end 71.29 42.51) (width 0.5) (layer "F.Cu") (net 4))
 (segment (start 86.45 50.12) (end 86.45 47.5) (width 0.5) (layer "F.Cu") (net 4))
 (segment (start 56.13 50.12) (end 56.13 47.5) (width 0.5) (layer "F.Cu") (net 4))
 (segment (start 101.61 50.12) (end 101.61 47.5) (width 0.5) (layer "F.Cu") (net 4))
 (segment (start 40.97 50.12) (end 40.97 47.5) (width 0.5) (layer "F.Cu") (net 4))
 (segment (start 71.3 42.5) (end 75.5 42.5) (width 0.5) (layer "F.Cu") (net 4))
 (segment (start 71.29 50.12) (end 71.29 47.5) (width 0.5) (layer "F.Cu") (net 4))
 (segment (start 71.29 42.51) (end 71.3 42.5) (width 0.5) (layer "F.Cu") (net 4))
 (via (at 86.45 47.5) (size 0.8) (drill 0.4) (layers "F.Cu" "B.Cu") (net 4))
 (via (at 75.5 42.5) (size 0.8) (drill 0.4) (layers "F.Cu" "B.Cu") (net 4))
 (via (at 101.61 47.5) (size 0.8) (drill 0.4) (layers "F.Cu" "B.Cu") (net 4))
 (via (at 56.13 47.5) (size 0.8) (drill 0.4) (layers "F.Cu" "B.Cu") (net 4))
 (via (at 40.97 47.5) (size 0.8) (drill 0.4) (layers "F.Cu" "B.Cu") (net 4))
 (via (at 71.29 47.5) (size 0.8) (drill 0.4) (layers "F.Cu" "B.Cu") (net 4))
 (segment (start 75.5 42.5) (end 73.83 42.5) (width 0.5) (layer "B.Cu") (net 4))
 (segment (start 40.97 47.5) (end 101.61 47.5) (width 0.5) (layer "B.Cu") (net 4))
 (segment (start 104.15 50.12) (end 104.15 46) (width 0.5) (layer "F.Cu") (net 5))
 (segment (start 58.67 50.12) (end 58.67 46) (width 0.5) (layer "F.Cu") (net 5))
 (segment (start 73.83 50.12) (end 73.83 46) (width 0.5) (layer "F.Cu") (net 5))
 (segment (start 88.99 50.12) (end 88.99 46) (width 0.5) (layer "F.Cu") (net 5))
 (segment (start 43.51 50.12) (end 43.51 46) (width 0.5) (layer "F.Cu") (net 5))
 (via (at 43.51 46) (size 0.8) (drill 0.4) (layers "F.Cu" "B.Cu") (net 5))
 (via (at 58.67 46) (size 0.8) (drill 0.4) (layers "F.Cu" "B.Cu") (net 5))
 (via (at 104.15 46) (size 0.8) (drill 0.4) (layers "F.Cu" "B.Cu") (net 5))
 (via (at 88.99 46) (size 0.8) (drill 0.4) (layers "F.Cu" "B.Cu") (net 5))
 (via (at 73.83 46) (size 0.8) (drill 0.4) (layers "F.Cu" "B.Cu") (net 5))
 (segment (start 81.25 46) (end 104.15 46) (width 0.5) (layer "B.Cu") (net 5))
 (segment (start 56.2 46) (end 81.25 46) (width 0.5) (layer "B.Cu") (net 5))
 (segment (start 56.13 45.93) (end 56.2 46) (width 0.5) (layer "B.Cu") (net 5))
 (segment (start 43.51 46) (end 56.2 46) (width 0.5) (layer "B.Cu") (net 5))
 (segment (start 56.13 42.5) (end 56.13 45.93) (width 0.5) (layer "B.Cu") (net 5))
 (segment (start 43.51 34.88) (end 43.51 39) (width 0.5) (layer "F.Cu") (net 6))
 (segment (start 73.83 34.88) (end 73.83 39) (width 0.5) (layer "F.Cu") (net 6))
 (segment (start 58.67 34.88) (end 58.67 39) (width 0.5) (layer "F.Cu") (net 6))
 (segment (start 88.99 34.88) (end 88.99 39) (width 0.5) (layer "F.Cu") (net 6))
 (segment (start 104.15 34.88) (end 104.15 39) (width 0.5) (layer "F.Cu") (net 6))
 (via (at 88.99 39) (size 0.8) (drill 0.4) (layers "F.Cu" "B.Cu") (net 6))
 (via (at 104.15 39) (size 0.8) (drill 0.4) (layers "F.Cu" "B.Cu") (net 6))
 (via (at 43.51 39) (size 0.8) (drill 0.4) (layers "F.Cu" "B.Cu") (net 6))
 (via (at 73.83 39) (size 0.8) (drill 0.4) (layers "F.Cu" "B.Cu") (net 6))
 (via (at 58.67 39) (size 0.8) (drill 0.4) (layers "F.Cu" "B.Cu") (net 6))
 (segment (start 78.9 39) (end 104.15 39) (width 0.5) (layer "B.Cu") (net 6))
 (segment (start 43.51 39) (end 78.9 39) (width 0.5) (layer "B.Cu") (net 6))
 (segment (start 78.83 42.5) (end 78.83 39.07) (width 0.5) (layer "B.Cu") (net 6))
 (segment (start 78.83 39.07) (end 78.9 39) (width 0.5) (layer "B.Cu") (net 6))
 (segment (start 71.29 34.88) (end 71.29 37.5) (width 0.5) (layer "F.Cu") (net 7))
 (segment (start 56.13 34.88) (end 56.13 37.5) (width 0.5) (layer "F.Cu") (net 7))
 (segment (start 81.37 40) (end 81.37 37.53) (width 0.5) (layer "F.Cu") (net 7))
 (segment (start 40.97 34.88) (end 40.97 37.5) (width 0.5) (layer "F.Cu") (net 7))
 (segment (start 86.45 34.88) (end 86.45 37.5) (width 0.5) (layer "F.Cu") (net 7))
 (segment (start 101.61 34.88) (end 101.61 37.5) (width 0.5) (layer "F.Cu") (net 7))
 (via (at 40.97 37.5) (size 0.8) (drill 0.4) (layers "F.Cu" "B.Cu") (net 7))
 (via (at 56.13 37.5) (size 0.8) (drill 0.4) (layers "F.Cu" "B.Cu") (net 7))
 (via (at 71.29 37.5) (size 0.8) (drill 0.4) (layers "F.Cu" "B.Cu") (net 7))
 (via (at 81.37 40) (size 0.8) (drill 0.4) (layers "F.Cu" "B.Cu") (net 7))
 (via (at 101.61 37.5) (size 0.8) (drill 0.4) (layers "F.Cu" "B.Cu") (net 7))
 (via (at 81.37 37.53) (size 0.8) (drill 0.4) (layers "F.Cu" "B.Cu") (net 7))
 (via (at 86.45 37.5) (size 0.8) (drill 0.4) (layers "F.Cu" "B.Cu") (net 7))
 (segment (start 81.37 42.5) (end 81.37 40) (width 0.5) (layer "B.Cu") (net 7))
 (segment (start 101.61 37.5) (end 40.97 37.5) (width 0.5) (layer "B.Cu") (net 7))
 (segment (start 66.21 34.88) (end 66.21 31) (width 0.5) (layer "F.Cu") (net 8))
 (segment (start 66.21 34.88) (end 66.21 40) (width 0.5) (layer "F.Cu") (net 8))
 (segment (start 81.37 34.88) (end 81.37 31) (width 0.5) (layer "F.Cu") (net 8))
 (segment (start 51.05 34.88) (end 51.05 31) (width 0.5) (layer "F.Cu") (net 8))
 (segment (start 63.67 40) (end 66.21 40) (width 0.5) (layer "F.Cu") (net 8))
 (segment (start 96.53 34.88) (end 96.53 31) (width 0.5) (layer "F.Cu") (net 8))
 (segment (start 35.89 34.88) (end 35.89 31) (width 0.5) (layer "F.Cu") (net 8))
 (via (at 63.67 40) (size 0.8) (drill 0.4) (layers "F.Cu" "B.Cu") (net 8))
 (via (at 96.53 31) (size 0.8) (drill 0.4) (layers "F.Cu" "B.Cu") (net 8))
 (via (at 35.89 31) (size 0.8) (drill 0.4) (layers "F.Cu" "B.Cu") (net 8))
 (via (at 66.21 31) (size 0.8) (drill 0.4) (layers "F.Cu" "B.Cu") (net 8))
 (via (at 51.05 31) (size 0.8) (drill 0.4) (layers "F.Cu" "B.Cu") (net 8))
 (via (at 81.37 31) (size 0.8) (drill 0.4) (layers "F.Cu" "B.Cu") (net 8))
 (segment (start 63.67 42.5) (end 63.67 40) (width 0.5) (layer "B.Cu") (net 8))
 (segment (start 35.89 31) (end 96.53 31) (width 0.5) (layer "B.Cu") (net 8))
 (segment (start 63.67 34.88) (end 60.67 34.88) (width 0.5) (layer "F.Cu") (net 9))
 (segment (start 78.83 34.88) (end 78.83 32.5) (width 0.5) (layer "F.Cu") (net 9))
 (segment (start 33.35 34.88) (end 33.35 32.5) (width 0.5) (layer "F.Cu") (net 9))
 (segment (start 48.51 34.88) (end 48.51 32.5) (width 0.5) (layer "F.Cu") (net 9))
 (segment (start 63.67 34.88) (end 63.67 32.5) (width 0.5) (layer "F.Cu") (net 9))
 (segment (start 93.99 32.5) (end 93.99 34.88) (width 0.5) (layer "F.Cu") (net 9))
 (segment (start 60.67 42.5) (end 60.67 34.88) (width 0.5) (layer "F.Cu") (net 9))
 (via (at 78.83 32.5) (size 0.8) (drill 0.4) (layers "F.Cu" "B.Cu") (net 9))
 (via (at 48.51 32.5) (size 0.8) (drill 0.4) (layers "F.Cu" "B.Cu") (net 9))
 (via (at 33.35 32.5) (size 0.8) (drill 0.4) (layers "F.Cu" "B.Cu") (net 9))
 (via (at 63.67 32.5) (size 0.8) (drill 0.4) (layers "F.Cu" "B.Cu") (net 9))
 (via (at 93.99 32.5) (size 0.8) (drill 0.4) (layers "F.Cu" "B.Cu") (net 9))
 (via (at 60.67 42.5) (size 0.8) (drill 0.4) (layers "F.Cu" "B.Cu") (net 9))
 (segment (start 58.67 42.5) (end 60.67 42.5) (width 0.5) (layer "B.Cu") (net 9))
 (segment (start 33.35 32.5) (end 93.99 32.5) (width 0.5) (layer "B.Cu") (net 9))
 (segment (start 53.59 42.41) (end 53.59 50.12) (width 0.5) (layer "F.Cu") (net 10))
 (segment (start 53.59 34.88) (end 53.59 42.41) (width 0.5) (layer "F.Cu") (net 10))
 (via (at 53.59 42.5) (size 1.5) (drill 0.75) (layers "F.Cu" "B.Cu") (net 10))
 (segment (start 68.75 42.5) (end 68.75 50.12) (width 0.5) (layer "F.Cu") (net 11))
 (segment (start 68.75 34.88) (end 68.75 42.5) (width 0.5) (layer "F.Cu") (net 11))
 (via (at 68.75 42.5) (size 1.5) (drill 0.75) (layers "F.Cu" "B.Cu") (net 11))
 (segment (start 83.91 34.88) (end 83.91 42.59) (width 0.5) (layer "F.Cu") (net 13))
 (segment (start 83.91 42.59) (end 83.91 50.12) (width 0.5) (layer "F.Cu") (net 13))
 (via (at 83.91 42.5) (size 1.5) (drill 0.75) (layers "F.Cu" "B.Cu") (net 13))
 (segment (start 99.07 34.88) (end 99.07 42.43) (width 0.5) (layer "F.Cu") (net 3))
 (segment (start 99.07 42.43) (end 99.07 50.12) (width 0.5) (layer "F.Cu") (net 3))
 (via (at 99.07 42.5) (size 1.5) (drill 0.75) (layers "F.Cu" "B.Cu") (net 3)))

